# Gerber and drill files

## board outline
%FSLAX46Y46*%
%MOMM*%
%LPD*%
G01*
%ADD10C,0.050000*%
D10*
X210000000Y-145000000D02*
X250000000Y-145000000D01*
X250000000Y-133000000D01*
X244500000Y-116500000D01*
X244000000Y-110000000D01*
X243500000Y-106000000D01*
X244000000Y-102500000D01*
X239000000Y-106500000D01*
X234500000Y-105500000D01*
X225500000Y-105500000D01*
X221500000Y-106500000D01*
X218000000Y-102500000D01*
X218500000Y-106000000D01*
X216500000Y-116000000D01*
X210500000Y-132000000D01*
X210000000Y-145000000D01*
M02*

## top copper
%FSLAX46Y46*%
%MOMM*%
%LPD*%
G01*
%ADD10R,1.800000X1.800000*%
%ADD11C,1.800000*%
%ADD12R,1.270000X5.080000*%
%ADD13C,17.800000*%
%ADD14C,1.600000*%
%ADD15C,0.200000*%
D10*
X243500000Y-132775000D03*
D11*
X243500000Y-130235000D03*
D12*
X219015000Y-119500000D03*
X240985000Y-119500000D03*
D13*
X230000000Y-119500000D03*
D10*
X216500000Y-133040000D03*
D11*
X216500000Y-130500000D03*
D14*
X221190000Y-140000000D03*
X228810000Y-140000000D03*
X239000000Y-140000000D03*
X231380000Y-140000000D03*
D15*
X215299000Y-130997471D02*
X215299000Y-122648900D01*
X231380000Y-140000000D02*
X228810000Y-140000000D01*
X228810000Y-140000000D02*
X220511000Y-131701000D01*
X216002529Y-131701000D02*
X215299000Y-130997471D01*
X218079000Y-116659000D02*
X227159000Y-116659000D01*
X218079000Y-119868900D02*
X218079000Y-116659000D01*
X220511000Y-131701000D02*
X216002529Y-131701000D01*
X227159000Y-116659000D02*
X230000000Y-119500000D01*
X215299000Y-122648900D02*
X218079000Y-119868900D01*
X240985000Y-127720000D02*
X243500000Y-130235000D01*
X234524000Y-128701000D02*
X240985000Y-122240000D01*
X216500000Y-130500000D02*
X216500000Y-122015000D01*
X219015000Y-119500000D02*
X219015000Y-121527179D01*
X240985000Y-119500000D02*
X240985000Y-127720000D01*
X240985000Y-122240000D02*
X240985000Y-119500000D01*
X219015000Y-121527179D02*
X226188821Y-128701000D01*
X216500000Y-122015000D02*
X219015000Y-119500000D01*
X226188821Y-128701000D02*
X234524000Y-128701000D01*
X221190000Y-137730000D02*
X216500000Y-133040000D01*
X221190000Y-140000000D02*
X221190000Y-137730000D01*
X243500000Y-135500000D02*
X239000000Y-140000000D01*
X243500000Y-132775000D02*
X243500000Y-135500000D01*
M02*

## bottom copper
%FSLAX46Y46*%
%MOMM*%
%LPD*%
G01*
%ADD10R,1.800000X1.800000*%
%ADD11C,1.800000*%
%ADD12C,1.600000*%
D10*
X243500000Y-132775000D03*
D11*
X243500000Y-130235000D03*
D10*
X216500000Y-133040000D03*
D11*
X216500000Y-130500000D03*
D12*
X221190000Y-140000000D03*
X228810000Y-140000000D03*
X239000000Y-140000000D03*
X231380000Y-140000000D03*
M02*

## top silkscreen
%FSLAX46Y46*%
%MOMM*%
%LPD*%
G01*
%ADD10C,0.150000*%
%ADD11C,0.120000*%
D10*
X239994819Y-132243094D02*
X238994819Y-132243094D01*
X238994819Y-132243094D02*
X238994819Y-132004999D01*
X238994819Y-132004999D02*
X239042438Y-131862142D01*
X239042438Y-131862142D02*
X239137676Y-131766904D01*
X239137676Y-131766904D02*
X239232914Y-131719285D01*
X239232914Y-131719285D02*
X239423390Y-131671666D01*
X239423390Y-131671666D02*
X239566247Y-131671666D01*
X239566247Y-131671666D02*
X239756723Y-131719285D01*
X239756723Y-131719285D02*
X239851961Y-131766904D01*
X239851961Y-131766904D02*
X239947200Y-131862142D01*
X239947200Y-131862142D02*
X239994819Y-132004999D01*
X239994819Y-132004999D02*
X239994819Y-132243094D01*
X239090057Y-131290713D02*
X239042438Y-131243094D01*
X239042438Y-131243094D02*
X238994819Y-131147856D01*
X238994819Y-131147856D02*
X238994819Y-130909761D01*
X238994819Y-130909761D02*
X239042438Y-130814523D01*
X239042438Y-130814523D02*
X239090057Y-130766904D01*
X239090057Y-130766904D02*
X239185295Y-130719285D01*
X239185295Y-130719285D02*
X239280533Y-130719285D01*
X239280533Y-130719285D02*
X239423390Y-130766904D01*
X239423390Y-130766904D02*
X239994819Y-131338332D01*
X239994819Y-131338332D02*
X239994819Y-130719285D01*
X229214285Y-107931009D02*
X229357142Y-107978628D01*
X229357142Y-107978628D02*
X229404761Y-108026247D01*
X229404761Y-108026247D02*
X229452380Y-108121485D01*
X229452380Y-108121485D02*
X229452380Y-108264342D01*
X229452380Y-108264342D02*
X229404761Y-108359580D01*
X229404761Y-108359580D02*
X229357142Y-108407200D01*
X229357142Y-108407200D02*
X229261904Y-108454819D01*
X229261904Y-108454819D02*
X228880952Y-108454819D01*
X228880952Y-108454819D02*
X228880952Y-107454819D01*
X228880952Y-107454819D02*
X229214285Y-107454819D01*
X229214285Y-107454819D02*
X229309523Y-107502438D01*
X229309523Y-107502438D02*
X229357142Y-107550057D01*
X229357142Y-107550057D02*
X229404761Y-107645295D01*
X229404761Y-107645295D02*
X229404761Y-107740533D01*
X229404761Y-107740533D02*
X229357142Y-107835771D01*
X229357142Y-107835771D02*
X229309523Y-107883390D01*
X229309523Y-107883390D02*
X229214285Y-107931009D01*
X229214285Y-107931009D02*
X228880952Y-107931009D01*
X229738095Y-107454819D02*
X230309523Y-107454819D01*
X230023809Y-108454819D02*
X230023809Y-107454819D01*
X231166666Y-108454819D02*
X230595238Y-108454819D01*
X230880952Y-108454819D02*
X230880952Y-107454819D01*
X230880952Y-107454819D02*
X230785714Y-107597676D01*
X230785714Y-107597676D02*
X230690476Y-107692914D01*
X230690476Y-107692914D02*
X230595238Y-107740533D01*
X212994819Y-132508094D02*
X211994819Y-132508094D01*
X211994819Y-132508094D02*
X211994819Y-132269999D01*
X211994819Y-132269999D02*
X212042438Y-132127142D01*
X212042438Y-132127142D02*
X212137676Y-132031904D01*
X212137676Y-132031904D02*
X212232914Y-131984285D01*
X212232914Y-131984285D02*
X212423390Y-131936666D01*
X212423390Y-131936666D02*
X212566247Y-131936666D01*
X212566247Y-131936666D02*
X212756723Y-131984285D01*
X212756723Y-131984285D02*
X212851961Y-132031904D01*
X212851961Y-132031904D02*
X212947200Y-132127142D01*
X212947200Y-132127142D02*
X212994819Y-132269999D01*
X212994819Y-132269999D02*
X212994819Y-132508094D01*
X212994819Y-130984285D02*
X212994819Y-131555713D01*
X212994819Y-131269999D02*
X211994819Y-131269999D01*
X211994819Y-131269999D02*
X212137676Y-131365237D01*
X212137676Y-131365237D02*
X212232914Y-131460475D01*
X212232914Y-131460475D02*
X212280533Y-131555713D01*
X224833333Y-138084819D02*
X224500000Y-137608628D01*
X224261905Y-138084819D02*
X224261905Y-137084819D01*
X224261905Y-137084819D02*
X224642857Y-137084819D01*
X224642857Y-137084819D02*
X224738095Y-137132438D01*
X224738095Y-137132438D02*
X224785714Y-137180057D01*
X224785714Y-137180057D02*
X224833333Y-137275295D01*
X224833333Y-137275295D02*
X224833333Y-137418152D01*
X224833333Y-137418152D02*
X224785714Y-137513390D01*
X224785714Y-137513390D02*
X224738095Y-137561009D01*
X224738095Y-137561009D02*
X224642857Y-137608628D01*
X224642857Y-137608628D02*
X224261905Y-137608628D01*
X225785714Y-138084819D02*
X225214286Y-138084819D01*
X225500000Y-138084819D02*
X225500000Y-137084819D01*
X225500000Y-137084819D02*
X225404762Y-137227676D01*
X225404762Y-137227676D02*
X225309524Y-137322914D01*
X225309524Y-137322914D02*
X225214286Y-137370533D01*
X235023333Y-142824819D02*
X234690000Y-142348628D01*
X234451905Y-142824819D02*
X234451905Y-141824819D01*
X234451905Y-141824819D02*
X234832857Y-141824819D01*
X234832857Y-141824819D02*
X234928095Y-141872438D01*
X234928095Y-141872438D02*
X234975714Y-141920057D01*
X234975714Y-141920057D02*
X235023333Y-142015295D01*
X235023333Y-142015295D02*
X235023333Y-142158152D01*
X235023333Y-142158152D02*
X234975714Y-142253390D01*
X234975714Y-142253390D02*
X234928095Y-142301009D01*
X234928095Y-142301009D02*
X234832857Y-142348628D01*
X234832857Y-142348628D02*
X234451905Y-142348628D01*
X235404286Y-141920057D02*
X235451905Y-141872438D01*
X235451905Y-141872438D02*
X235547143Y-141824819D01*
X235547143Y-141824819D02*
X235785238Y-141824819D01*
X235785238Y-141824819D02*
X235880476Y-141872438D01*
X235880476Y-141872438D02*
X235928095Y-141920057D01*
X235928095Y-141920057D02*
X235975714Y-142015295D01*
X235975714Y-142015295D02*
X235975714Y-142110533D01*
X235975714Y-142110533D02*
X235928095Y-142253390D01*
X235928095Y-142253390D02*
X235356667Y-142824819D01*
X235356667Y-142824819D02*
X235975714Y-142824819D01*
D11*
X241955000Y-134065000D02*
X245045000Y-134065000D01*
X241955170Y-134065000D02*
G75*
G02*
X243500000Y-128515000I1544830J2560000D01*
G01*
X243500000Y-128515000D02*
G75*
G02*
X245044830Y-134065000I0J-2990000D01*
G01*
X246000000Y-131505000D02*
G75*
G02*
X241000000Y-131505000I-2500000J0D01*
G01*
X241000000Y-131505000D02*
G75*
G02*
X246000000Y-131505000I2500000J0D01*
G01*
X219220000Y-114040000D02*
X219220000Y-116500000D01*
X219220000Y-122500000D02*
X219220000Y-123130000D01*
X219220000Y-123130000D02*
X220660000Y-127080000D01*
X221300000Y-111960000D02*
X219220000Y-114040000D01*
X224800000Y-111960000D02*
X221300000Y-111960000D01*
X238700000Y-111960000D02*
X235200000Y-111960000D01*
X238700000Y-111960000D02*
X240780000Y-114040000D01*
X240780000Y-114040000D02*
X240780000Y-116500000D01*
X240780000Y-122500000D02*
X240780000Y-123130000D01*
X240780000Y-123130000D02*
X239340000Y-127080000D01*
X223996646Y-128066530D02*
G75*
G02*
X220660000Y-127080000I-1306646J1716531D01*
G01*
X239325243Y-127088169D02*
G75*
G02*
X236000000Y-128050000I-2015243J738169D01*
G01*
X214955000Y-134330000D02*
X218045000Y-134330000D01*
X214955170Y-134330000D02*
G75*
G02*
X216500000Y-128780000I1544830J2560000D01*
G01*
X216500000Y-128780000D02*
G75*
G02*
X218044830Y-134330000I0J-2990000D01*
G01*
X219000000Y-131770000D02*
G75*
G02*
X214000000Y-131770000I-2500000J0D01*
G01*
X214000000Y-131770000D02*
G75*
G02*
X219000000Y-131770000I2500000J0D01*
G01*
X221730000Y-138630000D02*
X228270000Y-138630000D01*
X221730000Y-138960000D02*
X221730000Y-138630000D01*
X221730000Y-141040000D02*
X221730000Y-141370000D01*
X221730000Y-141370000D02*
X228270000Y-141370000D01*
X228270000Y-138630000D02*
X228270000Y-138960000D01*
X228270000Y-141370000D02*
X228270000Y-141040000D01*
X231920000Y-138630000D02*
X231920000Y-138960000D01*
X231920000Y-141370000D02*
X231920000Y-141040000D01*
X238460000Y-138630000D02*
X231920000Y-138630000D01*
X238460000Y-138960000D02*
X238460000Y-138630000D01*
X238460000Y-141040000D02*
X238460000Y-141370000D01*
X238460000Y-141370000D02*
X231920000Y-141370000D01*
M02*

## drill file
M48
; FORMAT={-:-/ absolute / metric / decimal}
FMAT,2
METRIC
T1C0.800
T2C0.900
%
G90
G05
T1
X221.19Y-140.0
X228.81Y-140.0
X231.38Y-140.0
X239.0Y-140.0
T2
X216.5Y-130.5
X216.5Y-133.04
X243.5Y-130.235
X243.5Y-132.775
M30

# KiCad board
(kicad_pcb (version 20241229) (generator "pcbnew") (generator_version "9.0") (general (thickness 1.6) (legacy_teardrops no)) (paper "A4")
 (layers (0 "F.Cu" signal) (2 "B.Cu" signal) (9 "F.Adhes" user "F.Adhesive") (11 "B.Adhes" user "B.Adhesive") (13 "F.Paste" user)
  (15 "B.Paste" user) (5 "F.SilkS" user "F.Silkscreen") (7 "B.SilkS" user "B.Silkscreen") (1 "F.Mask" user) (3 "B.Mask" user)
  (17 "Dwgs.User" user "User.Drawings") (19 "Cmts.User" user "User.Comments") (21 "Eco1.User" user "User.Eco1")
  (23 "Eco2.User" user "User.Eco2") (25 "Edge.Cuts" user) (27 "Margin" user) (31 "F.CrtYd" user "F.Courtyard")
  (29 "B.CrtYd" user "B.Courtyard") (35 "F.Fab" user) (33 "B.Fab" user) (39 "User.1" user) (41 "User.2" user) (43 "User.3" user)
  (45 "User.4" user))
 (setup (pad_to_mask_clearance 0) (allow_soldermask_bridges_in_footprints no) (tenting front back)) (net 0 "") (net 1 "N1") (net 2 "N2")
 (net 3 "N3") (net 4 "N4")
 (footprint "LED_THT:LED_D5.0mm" (layer "F.Cu") (at 243.5 132.775 90)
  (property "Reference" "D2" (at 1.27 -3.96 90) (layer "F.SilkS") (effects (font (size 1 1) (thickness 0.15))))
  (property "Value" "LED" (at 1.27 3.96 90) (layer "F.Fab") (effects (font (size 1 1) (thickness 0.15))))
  (fp_line (start -1.29 -1.545) (end -1.29 1.545) (stroke (width 0.12) (type solid)) (layer "F.SilkS"))
  (fp_arc (start -1.29 -1.54483) (mid 2.071779 -2.880495) (end 4.26 0) (stroke (width 0.12) (type solid)) (layer "F.SilkS"))
  (fp_arc (start 4.26 0) (mid 2.071779 2.880495) (end -1.29 1.54483) (stroke (width 0.12) (type solid)) (layer "F.SilkS"))
  (fp_circle (center 1.27 0) (end 3.77 0) (stroke (width 0.12) (type solid)) (fill no) (layer "F.SilkS"))
  (pad "1" thru_hole rect (at 0 0 90) (size 1.8 1.8) (drill 0.9) (layers "*.Cu" "*.Mask") (remove_unused_layers no) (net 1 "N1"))
  (pad "2" thru_hole circle (at 2.54 0 90) (size 1.8 1.8) (drill 0.9) (layers "*.Cu" "*.Mask") (remove_unused_layers no) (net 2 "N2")))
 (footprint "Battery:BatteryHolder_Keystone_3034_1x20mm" (layer "F.Cu") (at 230 119.5)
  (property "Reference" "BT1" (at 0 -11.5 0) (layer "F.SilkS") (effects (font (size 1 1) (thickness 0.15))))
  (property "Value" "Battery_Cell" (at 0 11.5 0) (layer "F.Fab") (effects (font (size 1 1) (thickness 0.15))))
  (fp_line (start -10.78 -5.46) (end -10.78 -3) (stroke (width 0.12) (type solid)) (layer "F.SilkS"))
  (fp_line (start -10.78 3) (end -10.78 3.63) (stroke (width 0.12) (type solid)) (layer "F.SilkS"))
  (fp_line (start -10.78 3.63) (end -9.34 7.58) (stroke (width 0.12) (type solid)) (layer "F.SilkS"))
  (fp_line (start -8.7 -7.54) (end -10.78 -5.46) (stroke (width 0.12) (type solid)) (layer "F.SilkS"))
  (fp_line (start -5.2 -7.54) (end -8.7 -7.54) (stroke (width 0.12) (type solid)) (layer "F.SilkS"))
  (fp_line (start 8.7 -7.54) (end 5.2 -7.54) (stroke (width 0.12) (type solid)) (layer "F.SilkS"))
  (fp_line (start 8.7 -7.54) (end 10.78 -5.46) (stroke (width 0.12) (type solid)) (layer "F.SilkS"))
  (fp_line (start 10.78 -5.46) (end 10.78 -3) (stroke (width 0.12) (type solid)) (layer "F.SilkS"))
  (fp_line (start 10.78 3) (end 10.78 3.63) (stroke (width 0.12) (type solid)) (layer "F.SilkS"))
  (fp_line (start 10.78 3.63) (end 9.34 7.58) (stroke (width 0.12) (type solid)) (layer "F.SilkS"))
  (fp_arc (start -6.003354 8.56653) (mid -7.921654 8.918738) (end -9.34 7.58) (stroke (width 0.12) (type solid)) (layer "F.SilkS"))
  (fp_arc (start 9.325243 7.588169) (mid 7.90634 8.911668) (end 6 8.55) (stroke (width 0.12) (type solid)) (layer "F.SilkS"))
  (pad "1" smd rect (at -10.985 0) (size 1.27 5.08) (layers "F.Cu" "F.Mask" "F.Paste") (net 2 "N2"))
  (pad "1" smd rect (at 10.985 0) (size 1.27 5.08) (layers "F.Cu" "F.Mask" "F.Paste") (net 2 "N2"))
  (pad "2" smd circle (at 0 0) (size 17.8 17.8) (layers "F.Cu" "F.Mask") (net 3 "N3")))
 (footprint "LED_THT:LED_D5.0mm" (layer "F.Cu") (at 216.5 133.04 90)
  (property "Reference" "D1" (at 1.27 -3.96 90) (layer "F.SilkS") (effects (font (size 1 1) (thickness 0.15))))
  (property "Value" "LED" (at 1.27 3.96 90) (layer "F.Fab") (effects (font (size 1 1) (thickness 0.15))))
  (fp_line (start -1.29 -1.545) (end -1.29 1.545) (stroke (width 0.12) (type solid)) (layer "F.SilkS"))
  (fp_arc (start -1.29 -1.54483) (mid 2.071779 -2.880495) (end 4.26 0) (stroke (width 0.12) (type solid)) (layer "F.SilkS"))
  (fp_arc (start 4.26 0) (mid 2.071779 2.880495) (end -1.29 1.54483) (stroke (width 0.12) (type solid)) (layer "F.SilkS"))
  (fp_circle (center 1.27 0) (end 3.77 0) (stroke (width 0.12) (type solid)) (fill no) (layer "F.SilkS"))
  (pad "1" thru_hole rect (at 0 0 90) (size 1.8 1.8) (drill 0.9) (layers "*.Cu" "*.Mask") (remove_unused_layers no) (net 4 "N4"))
  (pad "2" thru_hole circle (at 2.54 0 90) (size 1.8 1.8) (drill 0.9) (layers "*.Cu" "*.Mask") (remove_unused_layers no) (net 2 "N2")))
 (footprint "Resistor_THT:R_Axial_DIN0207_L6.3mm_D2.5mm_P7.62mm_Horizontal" (layer "F.Cu") (at 221.19 140)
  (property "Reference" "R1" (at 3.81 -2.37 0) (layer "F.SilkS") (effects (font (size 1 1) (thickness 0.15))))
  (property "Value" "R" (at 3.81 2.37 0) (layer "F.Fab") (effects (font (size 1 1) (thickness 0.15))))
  (fp_line (start 0.54 -1.37) (end 7.08 -1.37) (stroke (width 0.12) (type solid)) (layer "F.SilkS"))
  (fp_line (start 0.54 -1.04) (end 0.54 -1.37) (stroke (width 0.12) (type solid)) (layer "F.SilkS"))
  (fp_line (start 0.54 1.04) (end 0.54 1.37) (stroke (width 0.12) (type solid)) (layer "F.SilkS"))
  (fp_line (start 0.54 1.37) (end 7.08 1.37) (stroke (width 0.12) (type solid)) (layer "F.SilkS"))
  (fp_line (start 7.08 -1.37) (end 7.08 -1.04) (stroke (width 0.12) (type solid)) (layer "F.SilkS"))
  (fp_line (start 7.08 1.37) (end 7.08 1.04) (stroke (width 0.12) (type solid)) (layer "F.SilkS"))
  (pad "1" thru_hole circle (at 0 0) (size 1.6 1.6) (drill 0.8) (layers "*.Cu" "*.Mask") (remove_unused_layers no) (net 4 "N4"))
  (pad "2" thru_hole circle (at 7.62 0) (size 1.6 1.6) (drill 0.8) (layers "*.Cu" "*.Mask") (remove_unused_layers no) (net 3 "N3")))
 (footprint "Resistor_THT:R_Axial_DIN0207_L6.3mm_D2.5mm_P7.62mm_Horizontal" (layer "F.Cu") (at 239 140 180)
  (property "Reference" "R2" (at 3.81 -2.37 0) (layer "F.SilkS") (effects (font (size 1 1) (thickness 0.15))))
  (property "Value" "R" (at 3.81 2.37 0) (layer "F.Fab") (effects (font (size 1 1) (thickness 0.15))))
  (fp_line (start 7.08 1.37) (end 7.08 1.04) (stroke (width 0.12) (type solid)) (layer "F.SilkS"))
  (fp_line (start 7.08 -1.37) (end 7.08 -1.04) (stroke (width 0.12) (type solid)) (layer "F.SilkS"))
  (fp_line (start 0.54 1.37) (end 7.08 1.37) (stroke (width 0.12) (type solid)) (layer "F.SilkS"))
  (fp_line (start 0.54 1.04) (end 0.54 1.37) (stroke (width 0.12) (type solid)) (layer "F.SilkS"))
  (fp_line (start 0.54 -1.04) (end 0.54 -1.37) (stroke (width 0.12) (type solid)) (layer "F.SilkS"))
  (fp_line (start 0.54 -1.37) (end 7.08 -1.37) (stroke (width 0.12) (type solid)) (layer "F.SilkS"))
  (pad "1" thru_hole circle (at 0 0 180) (size 1.6 1.6) (drill 0.8) (layers "*.Cu" "*.Mask") (remove_unused_layers no) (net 1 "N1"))
  (pad "2" thru_hole circle (at 7.62 0 180) (size 1.6 1.6) (drill 0.8) (layers "*.Cu" "*.Mask") (remove_unused_layers no) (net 3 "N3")))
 (gr_poly
  (pts (xy 210 145) (xy 250 145) (xy 250 133) (xy 244.5 116.5) (xy 244 110) (xy 243.5 106) (xy 244 102.5) (xy 239 106.5) (xy 234.5 105.5)
   (xy 225.5 105.5) (xy 221.5 106.5) (xy 218 102.5) (xy 218.5 106) (xy 216.5 116) (xy 210.5 132))
  (stroke (width 0.05) (type solid)) (fill no) (layer "Edge.Cuts"))
 (segment (start 215.299 130.997471) (end 215.299 122.6489) (width 0.2) (layer "F.Cu") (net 3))
 (segment (start 231.38 140) (end 228.81 140) (width 0.2) (layer "F.Cu") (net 3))
 (segment (start 228.81 140) (end 220.511 131.701) (width 0.2) (layer "F.Cu") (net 3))
 (segment (start 216.002529 131.701) (end 215.299 130.997471) (width 0.2) (layer "F.Cu") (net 3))
 (segment (start 218.079 116.659) (end 227.159 116.659) (width 0.2) (layer "F.Cu") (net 3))
 (segment (start 218.079 119.8689) (end 218.079 116.659) (width 0.2) (layer "F.Cu") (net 3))
 (segment (start 220.511 131.701) (end 216.002529 131.701) (width 0.2) (layer "F.Cu") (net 3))
 (segment (start 227.159 116.659) (end 230 119.5) (width 0.2) (layer "F.Cu") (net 3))
 (segment (start 215.299 122.6489) (end 218.079 119.8689) (width 0.2) (layer "F.Cu") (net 3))
 (segment (start 240.985 127.72) (end 243.5 130.235) (width 0.2) (layer "F.Cu") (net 2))
 (segment (start 234.524 128.701) (end 240.985 122.24) (width 0.2) (layer "F.Cu") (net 2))
 (segment (start 216.5 130.5) (end 216.5 122.015) (width 0.2) (layer "F.Cu") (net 2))
 (segment (start 219.015 119.5) (end 219.015 121.527179) (width 0.2) (layer "F.Cu") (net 2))
 (segment (start 240.985 119.5) (end 240.985 127.72) (width 0.2) (layer "F.Cu") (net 2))
 (segment (start 240.985 122.24) (end 240.985 119.5) (width 0.2) (layer "F.Cu") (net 2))
 (segment (start 219.015 121.527179) (end 226.188821 128.701) (width 0.2) (layer "F.Cu") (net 2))
 (segment (start 216.5 122.015) (end 219.015 119.5) (width 0.2) (layer "F.Cu") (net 2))
 (segment (start 226.188821 128.701) (end 234.524 128.701) (width 0.2) (layer "F.Cu") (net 2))
 (segment (start 221.19 137.73) (end 216.5 133.04) (width 0.2) (layer "F.Cu") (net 4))
 (segment (start 221.19 140) (end 221.19 137.73) (width 0.2) (layer "F.Cu") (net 4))
 (segment (start 243.5 135.5) (end 239 140) (width 0.2) (layer "F.Cu") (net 1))
 (segment (start 243.5 132.775) (end 243.5 135.5) (width 0.2) (layer "F.Cu") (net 1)))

